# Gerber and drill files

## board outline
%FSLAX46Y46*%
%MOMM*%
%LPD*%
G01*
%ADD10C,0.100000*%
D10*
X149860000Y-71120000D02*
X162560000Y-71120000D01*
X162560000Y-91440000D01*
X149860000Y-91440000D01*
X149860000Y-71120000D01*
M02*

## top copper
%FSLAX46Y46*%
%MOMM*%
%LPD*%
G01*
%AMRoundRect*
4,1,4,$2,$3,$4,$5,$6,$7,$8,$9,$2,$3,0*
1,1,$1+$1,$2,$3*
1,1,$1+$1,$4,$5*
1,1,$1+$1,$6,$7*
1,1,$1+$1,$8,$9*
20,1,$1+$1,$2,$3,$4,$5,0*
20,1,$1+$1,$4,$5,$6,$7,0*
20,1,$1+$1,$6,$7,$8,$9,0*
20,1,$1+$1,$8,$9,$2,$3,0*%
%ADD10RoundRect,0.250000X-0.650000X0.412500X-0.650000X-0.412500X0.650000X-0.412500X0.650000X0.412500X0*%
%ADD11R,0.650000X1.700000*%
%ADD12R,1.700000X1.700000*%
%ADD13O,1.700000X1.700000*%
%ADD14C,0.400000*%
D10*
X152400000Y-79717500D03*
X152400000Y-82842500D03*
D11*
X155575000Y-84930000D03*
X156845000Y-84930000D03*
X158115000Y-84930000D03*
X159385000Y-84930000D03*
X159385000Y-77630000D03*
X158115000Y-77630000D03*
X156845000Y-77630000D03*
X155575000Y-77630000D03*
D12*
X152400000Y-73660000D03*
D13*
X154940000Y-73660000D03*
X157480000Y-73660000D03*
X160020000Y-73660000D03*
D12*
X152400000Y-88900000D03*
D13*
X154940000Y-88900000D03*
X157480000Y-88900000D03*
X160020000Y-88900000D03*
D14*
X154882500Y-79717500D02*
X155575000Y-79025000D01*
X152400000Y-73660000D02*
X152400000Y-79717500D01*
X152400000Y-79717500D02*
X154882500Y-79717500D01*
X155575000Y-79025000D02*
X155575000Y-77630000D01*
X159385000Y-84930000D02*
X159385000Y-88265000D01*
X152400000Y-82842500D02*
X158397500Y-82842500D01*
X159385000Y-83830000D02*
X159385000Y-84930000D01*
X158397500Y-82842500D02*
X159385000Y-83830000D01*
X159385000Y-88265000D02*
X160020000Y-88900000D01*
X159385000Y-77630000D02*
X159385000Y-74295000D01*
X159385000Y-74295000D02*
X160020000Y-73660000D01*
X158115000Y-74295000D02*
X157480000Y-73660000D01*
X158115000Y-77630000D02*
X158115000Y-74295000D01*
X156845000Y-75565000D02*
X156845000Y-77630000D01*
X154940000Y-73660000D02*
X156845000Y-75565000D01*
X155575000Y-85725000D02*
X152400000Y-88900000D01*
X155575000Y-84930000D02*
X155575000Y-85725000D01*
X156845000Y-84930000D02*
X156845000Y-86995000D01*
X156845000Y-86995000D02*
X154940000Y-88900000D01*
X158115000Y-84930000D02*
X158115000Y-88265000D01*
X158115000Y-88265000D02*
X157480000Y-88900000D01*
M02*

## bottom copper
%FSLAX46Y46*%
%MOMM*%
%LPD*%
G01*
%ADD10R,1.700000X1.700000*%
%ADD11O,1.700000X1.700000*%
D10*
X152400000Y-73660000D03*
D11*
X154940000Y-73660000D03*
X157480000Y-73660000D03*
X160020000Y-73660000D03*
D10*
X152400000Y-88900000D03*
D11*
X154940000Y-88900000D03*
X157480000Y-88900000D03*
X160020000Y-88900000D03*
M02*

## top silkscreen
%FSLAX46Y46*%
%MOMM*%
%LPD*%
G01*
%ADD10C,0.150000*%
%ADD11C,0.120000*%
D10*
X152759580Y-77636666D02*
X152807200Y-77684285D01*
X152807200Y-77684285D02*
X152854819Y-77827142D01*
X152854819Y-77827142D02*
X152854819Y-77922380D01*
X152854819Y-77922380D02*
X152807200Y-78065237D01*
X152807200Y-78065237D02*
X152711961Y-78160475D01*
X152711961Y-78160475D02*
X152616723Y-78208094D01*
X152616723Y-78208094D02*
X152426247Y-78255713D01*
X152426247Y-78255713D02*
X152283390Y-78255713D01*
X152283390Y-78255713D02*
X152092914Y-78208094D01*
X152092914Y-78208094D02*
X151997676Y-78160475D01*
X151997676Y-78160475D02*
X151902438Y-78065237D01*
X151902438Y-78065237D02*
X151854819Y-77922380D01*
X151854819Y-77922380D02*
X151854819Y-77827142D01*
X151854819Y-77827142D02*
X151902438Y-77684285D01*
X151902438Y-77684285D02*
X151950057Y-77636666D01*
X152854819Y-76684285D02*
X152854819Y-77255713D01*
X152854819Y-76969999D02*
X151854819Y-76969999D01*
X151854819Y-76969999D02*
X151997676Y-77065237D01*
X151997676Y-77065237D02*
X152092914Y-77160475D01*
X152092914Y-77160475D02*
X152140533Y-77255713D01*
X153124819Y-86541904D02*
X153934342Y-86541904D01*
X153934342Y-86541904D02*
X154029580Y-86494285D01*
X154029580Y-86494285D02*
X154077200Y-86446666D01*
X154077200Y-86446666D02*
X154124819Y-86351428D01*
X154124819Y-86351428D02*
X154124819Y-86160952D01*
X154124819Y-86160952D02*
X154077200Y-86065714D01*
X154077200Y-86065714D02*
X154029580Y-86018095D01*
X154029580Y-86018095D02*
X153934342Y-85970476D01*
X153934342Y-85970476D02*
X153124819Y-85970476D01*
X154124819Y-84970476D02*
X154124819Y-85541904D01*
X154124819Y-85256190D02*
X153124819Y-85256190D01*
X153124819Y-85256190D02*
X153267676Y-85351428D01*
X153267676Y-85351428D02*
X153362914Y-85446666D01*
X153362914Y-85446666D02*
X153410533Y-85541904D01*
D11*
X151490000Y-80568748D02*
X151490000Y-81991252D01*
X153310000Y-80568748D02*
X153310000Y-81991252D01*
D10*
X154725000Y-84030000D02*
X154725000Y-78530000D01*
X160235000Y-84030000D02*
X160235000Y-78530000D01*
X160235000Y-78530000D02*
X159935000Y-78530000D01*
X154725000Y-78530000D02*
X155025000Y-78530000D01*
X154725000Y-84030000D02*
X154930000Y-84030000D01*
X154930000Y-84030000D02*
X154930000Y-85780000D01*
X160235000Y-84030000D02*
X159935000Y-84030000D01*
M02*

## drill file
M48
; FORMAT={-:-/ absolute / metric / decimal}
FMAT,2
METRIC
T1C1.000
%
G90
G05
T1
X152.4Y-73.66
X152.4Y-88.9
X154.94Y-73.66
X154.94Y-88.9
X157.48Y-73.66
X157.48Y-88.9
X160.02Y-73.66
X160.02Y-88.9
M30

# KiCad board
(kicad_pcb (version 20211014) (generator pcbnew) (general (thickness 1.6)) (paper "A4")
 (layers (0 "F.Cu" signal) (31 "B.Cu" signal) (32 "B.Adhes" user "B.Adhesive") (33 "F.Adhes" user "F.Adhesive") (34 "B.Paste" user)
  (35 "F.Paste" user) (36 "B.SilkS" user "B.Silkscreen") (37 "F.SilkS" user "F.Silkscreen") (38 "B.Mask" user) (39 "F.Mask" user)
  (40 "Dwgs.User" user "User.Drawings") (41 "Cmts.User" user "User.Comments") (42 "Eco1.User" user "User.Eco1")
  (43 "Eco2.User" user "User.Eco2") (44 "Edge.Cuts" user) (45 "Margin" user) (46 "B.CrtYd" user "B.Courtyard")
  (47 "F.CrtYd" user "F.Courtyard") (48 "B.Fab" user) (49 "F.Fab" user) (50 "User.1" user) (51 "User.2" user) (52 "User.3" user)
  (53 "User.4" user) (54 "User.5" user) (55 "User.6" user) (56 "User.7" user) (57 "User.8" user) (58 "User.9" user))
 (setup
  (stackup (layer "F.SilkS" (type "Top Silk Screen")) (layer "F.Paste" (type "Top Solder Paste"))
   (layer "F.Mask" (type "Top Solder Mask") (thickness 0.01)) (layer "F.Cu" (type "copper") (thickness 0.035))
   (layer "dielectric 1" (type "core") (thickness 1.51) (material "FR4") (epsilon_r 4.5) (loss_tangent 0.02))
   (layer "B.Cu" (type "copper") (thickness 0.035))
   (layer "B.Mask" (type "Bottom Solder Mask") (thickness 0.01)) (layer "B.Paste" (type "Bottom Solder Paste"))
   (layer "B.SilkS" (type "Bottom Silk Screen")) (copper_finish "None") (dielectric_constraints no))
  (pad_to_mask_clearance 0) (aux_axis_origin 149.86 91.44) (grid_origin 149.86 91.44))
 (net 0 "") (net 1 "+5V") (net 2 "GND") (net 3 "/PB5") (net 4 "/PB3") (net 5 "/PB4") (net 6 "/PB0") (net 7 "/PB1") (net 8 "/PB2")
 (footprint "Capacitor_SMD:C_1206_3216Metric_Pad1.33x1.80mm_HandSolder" (layer "F.Cu") (at 152.4 81.28 -90)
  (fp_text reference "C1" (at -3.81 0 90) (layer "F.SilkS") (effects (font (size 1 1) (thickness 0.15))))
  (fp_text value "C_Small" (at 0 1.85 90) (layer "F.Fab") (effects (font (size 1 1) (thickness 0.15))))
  (fp_line (start -0.711252 0.91) (end 0.711252 0.91) (layer "F.SilkS") (width 0.12))
  (fp_line (start -0.711252 -0.91) (end 0.711252 -0.91) (layer "F.SilkS") (width 0.12))
  (pad "1" smd roundrect (at -1.5625 0 270) (size 1.325 1.8) (layers "F.Cu" "F.Paste" "F.Mask") (roundrect_rratio 0.1886792453)
   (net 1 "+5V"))
  (pad "2" smd roundrect (at 1.5625 0 270) (size 1.325 1.8) (layers "F.Cu" "F.Paste" "F.Mask") (roundrect_rratio 0.1886792453) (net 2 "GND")))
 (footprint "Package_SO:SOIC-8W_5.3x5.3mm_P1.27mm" (layer "F.Cu") (at 157.48 81.28 90)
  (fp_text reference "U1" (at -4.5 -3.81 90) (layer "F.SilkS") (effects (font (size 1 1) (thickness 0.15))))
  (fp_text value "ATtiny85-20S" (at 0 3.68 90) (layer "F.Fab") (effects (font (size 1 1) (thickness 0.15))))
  (fp_line (start -2.75 -2.755) (end 2.75 -2.755) (layer "F.SilkS") (width 0.15))
  (fp_line (start -2.75 2.755) (end 2.75 2.755) (layer "F.SilkS") (width 0.15))
  (fp_line (start 2.75 2.755) (end 2.75 2.455) (layer "F.SilkS") (width 0.15))
  (fp_line (start 2.75 -2.755) (end 2.75 -2.455) (layer "F.SilkS") (width 0.15))
  (fp_line (start -2.75 -2.755) (end -2.75 -2.55) (layer "F.SilkS") (width 0.15))
  (fp_line (start -2.75 -2.55) (end -4.5 -2.55) (layer "F.SilkS") (width 0.15))
  (fp_line (start -2.75 2.755) (end -2.75 2.455) (layer "F.SilkS") (width 0.15))
  (pad "1" smd rect (at -3.65 -1.905 90) (size 1.7 0.65) (layers "F.Cu" "F.Paste" "F.Mask") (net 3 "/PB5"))
  (pad "2" smd rect (at -3.65 -0.635 90) (size 1.7 0.65) (layers "F.Cu" "F.Paste" "F.Mask") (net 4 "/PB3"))
  (pad "3" smd rect (at -3.65 0.635 90) (size 1.7 0.65) (layers "F.Cu" "F.Paste" "F.Mask") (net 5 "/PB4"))
  (pad "4" smd rect (at -3.65 1.905 90) (size 1.7 0.65) (layers "F.Cu" "F.Paste" "F.Mask") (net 2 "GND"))
  (pad "5" smd rect (at 3.65 1.905 90) (size 1.7 0.65) (layers "F.Cu" "F.Paste" "F.Mask") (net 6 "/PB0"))
  (pad "6" smd rect (at 3.65 0.635 90) (size 1.7 0.65) (layers "F.Cu" "F.Paste" "F.Mask") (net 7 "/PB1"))
  (pad "7" smd rect (at 3.65 -0.635 90) (size 1.7 0.65) (layers "F.Cu" "F.Paste" "F.Mask") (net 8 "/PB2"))
  (pad "8" smd rect (at 3.65 -1.905 90) (size 1.7 0.65) (layers "F.Cu" "F.Paste" "F.Mask") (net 1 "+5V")))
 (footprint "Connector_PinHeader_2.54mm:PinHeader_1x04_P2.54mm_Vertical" (layer "B.Cu") (at 152.4 73.66 -90)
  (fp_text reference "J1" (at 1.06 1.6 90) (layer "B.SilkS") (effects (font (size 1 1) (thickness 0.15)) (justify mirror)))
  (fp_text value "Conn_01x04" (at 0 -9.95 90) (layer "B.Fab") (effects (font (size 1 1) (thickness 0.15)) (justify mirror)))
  (pad "1" thru_hole rect (at 0 0 270) (size 1.7 1.7) (drill 1) (layers *.Cu *.Mask) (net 1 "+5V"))
  (pad "2" thru_hole oval (at 0 -2.54 270) (size 1.7 1.7) (drill 1) (layers *.Cu *.Mask) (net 8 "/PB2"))
  (pad "3" thru_hole oval (at 0 -5.08 270) (size 1.7 1.7) (drill 1) (layers *.Cu *.Mask) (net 7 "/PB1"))
  (pad "4" thru_hole oval (at 0 -7.62 270) (size 1.7 1.7) (drill 1) (layers *.Cu *.Mask) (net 6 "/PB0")))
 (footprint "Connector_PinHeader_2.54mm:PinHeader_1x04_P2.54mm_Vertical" (layer "B.Cu") (at 152.4 88.9 -90)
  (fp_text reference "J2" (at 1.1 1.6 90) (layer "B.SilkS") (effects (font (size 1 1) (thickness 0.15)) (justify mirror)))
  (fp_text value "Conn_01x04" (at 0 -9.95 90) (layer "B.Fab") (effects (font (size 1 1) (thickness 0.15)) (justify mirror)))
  (pad "1" thru_hole rect (at 0 0 270) (size 1.7 1.7) (drill 1) (layers *.Cu *.Mask) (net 3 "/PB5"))
  (pad "2" thru_hole oval (at 0 -2.54 270) (size 1.7 1.7) (drill 1) (layers *.Cu *.Mask) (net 4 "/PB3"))
  (pad "3" thru_hole oval (at 0 -5.08 270) (size 1.7 1.7) (drill 1) (layers *.Cu *.Mask) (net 5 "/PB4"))
  (pad "4" thru_hole oval (at 0 -7.62 270) (size 1.7 1.7) (drill 1) (layers *.Cu *.Mask) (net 2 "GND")))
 (gr_rect (start 149.86 91.44) (end 162.56 71.12) (layer "Edge.Cuts") (width 0.1) (fill none))
 (segment (start 154.8825 79.7175) (end 155.575 79.025) (width 0.4) (layer "F.Cu") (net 1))
 (segment (start 152.4 73.66) (end 152.4 79.7175) (width 0.4) (layer "F.Cu") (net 1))
 (segment (start 152.4 79.7175) (end 154.8825 79.7175) (width 0.4) (layer "F.Cu") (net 1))
 (segment (start 155.575 79.025) (end 155.575 77.63) (width 0.4) (layer "F.Cu") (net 1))
 (segment (start 159.385 84.93) (end 159.385 88.265) (width 0.4) (layer "F.Cu") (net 2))
 (segment (start 152.4 82.8425) (end 158.3975 82.8425) (width 0.4) (layer "F.Cu") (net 2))
 (segment (start 159.385 83.83) (end 159.385 84.93) (width 0.4) (layer "F.Cu") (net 2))
 (segment (start 158.3975 82.8425) (end 159.385 83.83) (width 0.4) (layer "F.Cu") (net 2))
 (segment (start 159.385 88.265) (end 160.02 88.9) (width 0.4) (layer "F.Cu") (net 2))
 (segment (start 159.385 77.63) (end 159.385 74.295) (width 0.4) (layer "F.Cu") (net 6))
 (segment (start 159.385 74.295) (end 160.02 73.66) (width 0.4) (layer "F.Cu") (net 6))
 (segment (start 158.115 74.295) (end 157.48 73.66) (width 0.4) (layer "F.Cu") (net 7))
 (segment (start 158.115 77.63) (end 158.115 74.295) (width 0.4) (layer "F.Cu") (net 7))
 (segment (start 156.845 75.565) (end 156.845 77.63) (width 0.4) (layer "F.Cu") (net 8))
 (segment (start 154.94 73.66) (end 156.845 75.565) (width 0.4) (layer "F.Cu") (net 8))
 (segment (start 155.575 85.725) (end 152.4 88.9) (width 0.4) (layer "F.Cu") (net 3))
 (segment (start 155.575 84.93) (end 155.575 85.725) (width 0.4) (layer "F.Cu") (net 3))
 (segment (start 156.845 84.93) (end 156.845 86.995) (width 0.4) (layer "F.Cu") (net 4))
 (segment (start 156.845 86.995) (end 154.94 88.9) (width 0.4) (layer "F.Cu") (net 4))
 (segment (start 158.115 84.93) (end 158.115 88.265) (width 0.4) (layer "F.Cu") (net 5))
 (segment (start 158.115 88.265) (end 157.48 88.9) (width 0.4) (layer "F.Cu") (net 5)))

